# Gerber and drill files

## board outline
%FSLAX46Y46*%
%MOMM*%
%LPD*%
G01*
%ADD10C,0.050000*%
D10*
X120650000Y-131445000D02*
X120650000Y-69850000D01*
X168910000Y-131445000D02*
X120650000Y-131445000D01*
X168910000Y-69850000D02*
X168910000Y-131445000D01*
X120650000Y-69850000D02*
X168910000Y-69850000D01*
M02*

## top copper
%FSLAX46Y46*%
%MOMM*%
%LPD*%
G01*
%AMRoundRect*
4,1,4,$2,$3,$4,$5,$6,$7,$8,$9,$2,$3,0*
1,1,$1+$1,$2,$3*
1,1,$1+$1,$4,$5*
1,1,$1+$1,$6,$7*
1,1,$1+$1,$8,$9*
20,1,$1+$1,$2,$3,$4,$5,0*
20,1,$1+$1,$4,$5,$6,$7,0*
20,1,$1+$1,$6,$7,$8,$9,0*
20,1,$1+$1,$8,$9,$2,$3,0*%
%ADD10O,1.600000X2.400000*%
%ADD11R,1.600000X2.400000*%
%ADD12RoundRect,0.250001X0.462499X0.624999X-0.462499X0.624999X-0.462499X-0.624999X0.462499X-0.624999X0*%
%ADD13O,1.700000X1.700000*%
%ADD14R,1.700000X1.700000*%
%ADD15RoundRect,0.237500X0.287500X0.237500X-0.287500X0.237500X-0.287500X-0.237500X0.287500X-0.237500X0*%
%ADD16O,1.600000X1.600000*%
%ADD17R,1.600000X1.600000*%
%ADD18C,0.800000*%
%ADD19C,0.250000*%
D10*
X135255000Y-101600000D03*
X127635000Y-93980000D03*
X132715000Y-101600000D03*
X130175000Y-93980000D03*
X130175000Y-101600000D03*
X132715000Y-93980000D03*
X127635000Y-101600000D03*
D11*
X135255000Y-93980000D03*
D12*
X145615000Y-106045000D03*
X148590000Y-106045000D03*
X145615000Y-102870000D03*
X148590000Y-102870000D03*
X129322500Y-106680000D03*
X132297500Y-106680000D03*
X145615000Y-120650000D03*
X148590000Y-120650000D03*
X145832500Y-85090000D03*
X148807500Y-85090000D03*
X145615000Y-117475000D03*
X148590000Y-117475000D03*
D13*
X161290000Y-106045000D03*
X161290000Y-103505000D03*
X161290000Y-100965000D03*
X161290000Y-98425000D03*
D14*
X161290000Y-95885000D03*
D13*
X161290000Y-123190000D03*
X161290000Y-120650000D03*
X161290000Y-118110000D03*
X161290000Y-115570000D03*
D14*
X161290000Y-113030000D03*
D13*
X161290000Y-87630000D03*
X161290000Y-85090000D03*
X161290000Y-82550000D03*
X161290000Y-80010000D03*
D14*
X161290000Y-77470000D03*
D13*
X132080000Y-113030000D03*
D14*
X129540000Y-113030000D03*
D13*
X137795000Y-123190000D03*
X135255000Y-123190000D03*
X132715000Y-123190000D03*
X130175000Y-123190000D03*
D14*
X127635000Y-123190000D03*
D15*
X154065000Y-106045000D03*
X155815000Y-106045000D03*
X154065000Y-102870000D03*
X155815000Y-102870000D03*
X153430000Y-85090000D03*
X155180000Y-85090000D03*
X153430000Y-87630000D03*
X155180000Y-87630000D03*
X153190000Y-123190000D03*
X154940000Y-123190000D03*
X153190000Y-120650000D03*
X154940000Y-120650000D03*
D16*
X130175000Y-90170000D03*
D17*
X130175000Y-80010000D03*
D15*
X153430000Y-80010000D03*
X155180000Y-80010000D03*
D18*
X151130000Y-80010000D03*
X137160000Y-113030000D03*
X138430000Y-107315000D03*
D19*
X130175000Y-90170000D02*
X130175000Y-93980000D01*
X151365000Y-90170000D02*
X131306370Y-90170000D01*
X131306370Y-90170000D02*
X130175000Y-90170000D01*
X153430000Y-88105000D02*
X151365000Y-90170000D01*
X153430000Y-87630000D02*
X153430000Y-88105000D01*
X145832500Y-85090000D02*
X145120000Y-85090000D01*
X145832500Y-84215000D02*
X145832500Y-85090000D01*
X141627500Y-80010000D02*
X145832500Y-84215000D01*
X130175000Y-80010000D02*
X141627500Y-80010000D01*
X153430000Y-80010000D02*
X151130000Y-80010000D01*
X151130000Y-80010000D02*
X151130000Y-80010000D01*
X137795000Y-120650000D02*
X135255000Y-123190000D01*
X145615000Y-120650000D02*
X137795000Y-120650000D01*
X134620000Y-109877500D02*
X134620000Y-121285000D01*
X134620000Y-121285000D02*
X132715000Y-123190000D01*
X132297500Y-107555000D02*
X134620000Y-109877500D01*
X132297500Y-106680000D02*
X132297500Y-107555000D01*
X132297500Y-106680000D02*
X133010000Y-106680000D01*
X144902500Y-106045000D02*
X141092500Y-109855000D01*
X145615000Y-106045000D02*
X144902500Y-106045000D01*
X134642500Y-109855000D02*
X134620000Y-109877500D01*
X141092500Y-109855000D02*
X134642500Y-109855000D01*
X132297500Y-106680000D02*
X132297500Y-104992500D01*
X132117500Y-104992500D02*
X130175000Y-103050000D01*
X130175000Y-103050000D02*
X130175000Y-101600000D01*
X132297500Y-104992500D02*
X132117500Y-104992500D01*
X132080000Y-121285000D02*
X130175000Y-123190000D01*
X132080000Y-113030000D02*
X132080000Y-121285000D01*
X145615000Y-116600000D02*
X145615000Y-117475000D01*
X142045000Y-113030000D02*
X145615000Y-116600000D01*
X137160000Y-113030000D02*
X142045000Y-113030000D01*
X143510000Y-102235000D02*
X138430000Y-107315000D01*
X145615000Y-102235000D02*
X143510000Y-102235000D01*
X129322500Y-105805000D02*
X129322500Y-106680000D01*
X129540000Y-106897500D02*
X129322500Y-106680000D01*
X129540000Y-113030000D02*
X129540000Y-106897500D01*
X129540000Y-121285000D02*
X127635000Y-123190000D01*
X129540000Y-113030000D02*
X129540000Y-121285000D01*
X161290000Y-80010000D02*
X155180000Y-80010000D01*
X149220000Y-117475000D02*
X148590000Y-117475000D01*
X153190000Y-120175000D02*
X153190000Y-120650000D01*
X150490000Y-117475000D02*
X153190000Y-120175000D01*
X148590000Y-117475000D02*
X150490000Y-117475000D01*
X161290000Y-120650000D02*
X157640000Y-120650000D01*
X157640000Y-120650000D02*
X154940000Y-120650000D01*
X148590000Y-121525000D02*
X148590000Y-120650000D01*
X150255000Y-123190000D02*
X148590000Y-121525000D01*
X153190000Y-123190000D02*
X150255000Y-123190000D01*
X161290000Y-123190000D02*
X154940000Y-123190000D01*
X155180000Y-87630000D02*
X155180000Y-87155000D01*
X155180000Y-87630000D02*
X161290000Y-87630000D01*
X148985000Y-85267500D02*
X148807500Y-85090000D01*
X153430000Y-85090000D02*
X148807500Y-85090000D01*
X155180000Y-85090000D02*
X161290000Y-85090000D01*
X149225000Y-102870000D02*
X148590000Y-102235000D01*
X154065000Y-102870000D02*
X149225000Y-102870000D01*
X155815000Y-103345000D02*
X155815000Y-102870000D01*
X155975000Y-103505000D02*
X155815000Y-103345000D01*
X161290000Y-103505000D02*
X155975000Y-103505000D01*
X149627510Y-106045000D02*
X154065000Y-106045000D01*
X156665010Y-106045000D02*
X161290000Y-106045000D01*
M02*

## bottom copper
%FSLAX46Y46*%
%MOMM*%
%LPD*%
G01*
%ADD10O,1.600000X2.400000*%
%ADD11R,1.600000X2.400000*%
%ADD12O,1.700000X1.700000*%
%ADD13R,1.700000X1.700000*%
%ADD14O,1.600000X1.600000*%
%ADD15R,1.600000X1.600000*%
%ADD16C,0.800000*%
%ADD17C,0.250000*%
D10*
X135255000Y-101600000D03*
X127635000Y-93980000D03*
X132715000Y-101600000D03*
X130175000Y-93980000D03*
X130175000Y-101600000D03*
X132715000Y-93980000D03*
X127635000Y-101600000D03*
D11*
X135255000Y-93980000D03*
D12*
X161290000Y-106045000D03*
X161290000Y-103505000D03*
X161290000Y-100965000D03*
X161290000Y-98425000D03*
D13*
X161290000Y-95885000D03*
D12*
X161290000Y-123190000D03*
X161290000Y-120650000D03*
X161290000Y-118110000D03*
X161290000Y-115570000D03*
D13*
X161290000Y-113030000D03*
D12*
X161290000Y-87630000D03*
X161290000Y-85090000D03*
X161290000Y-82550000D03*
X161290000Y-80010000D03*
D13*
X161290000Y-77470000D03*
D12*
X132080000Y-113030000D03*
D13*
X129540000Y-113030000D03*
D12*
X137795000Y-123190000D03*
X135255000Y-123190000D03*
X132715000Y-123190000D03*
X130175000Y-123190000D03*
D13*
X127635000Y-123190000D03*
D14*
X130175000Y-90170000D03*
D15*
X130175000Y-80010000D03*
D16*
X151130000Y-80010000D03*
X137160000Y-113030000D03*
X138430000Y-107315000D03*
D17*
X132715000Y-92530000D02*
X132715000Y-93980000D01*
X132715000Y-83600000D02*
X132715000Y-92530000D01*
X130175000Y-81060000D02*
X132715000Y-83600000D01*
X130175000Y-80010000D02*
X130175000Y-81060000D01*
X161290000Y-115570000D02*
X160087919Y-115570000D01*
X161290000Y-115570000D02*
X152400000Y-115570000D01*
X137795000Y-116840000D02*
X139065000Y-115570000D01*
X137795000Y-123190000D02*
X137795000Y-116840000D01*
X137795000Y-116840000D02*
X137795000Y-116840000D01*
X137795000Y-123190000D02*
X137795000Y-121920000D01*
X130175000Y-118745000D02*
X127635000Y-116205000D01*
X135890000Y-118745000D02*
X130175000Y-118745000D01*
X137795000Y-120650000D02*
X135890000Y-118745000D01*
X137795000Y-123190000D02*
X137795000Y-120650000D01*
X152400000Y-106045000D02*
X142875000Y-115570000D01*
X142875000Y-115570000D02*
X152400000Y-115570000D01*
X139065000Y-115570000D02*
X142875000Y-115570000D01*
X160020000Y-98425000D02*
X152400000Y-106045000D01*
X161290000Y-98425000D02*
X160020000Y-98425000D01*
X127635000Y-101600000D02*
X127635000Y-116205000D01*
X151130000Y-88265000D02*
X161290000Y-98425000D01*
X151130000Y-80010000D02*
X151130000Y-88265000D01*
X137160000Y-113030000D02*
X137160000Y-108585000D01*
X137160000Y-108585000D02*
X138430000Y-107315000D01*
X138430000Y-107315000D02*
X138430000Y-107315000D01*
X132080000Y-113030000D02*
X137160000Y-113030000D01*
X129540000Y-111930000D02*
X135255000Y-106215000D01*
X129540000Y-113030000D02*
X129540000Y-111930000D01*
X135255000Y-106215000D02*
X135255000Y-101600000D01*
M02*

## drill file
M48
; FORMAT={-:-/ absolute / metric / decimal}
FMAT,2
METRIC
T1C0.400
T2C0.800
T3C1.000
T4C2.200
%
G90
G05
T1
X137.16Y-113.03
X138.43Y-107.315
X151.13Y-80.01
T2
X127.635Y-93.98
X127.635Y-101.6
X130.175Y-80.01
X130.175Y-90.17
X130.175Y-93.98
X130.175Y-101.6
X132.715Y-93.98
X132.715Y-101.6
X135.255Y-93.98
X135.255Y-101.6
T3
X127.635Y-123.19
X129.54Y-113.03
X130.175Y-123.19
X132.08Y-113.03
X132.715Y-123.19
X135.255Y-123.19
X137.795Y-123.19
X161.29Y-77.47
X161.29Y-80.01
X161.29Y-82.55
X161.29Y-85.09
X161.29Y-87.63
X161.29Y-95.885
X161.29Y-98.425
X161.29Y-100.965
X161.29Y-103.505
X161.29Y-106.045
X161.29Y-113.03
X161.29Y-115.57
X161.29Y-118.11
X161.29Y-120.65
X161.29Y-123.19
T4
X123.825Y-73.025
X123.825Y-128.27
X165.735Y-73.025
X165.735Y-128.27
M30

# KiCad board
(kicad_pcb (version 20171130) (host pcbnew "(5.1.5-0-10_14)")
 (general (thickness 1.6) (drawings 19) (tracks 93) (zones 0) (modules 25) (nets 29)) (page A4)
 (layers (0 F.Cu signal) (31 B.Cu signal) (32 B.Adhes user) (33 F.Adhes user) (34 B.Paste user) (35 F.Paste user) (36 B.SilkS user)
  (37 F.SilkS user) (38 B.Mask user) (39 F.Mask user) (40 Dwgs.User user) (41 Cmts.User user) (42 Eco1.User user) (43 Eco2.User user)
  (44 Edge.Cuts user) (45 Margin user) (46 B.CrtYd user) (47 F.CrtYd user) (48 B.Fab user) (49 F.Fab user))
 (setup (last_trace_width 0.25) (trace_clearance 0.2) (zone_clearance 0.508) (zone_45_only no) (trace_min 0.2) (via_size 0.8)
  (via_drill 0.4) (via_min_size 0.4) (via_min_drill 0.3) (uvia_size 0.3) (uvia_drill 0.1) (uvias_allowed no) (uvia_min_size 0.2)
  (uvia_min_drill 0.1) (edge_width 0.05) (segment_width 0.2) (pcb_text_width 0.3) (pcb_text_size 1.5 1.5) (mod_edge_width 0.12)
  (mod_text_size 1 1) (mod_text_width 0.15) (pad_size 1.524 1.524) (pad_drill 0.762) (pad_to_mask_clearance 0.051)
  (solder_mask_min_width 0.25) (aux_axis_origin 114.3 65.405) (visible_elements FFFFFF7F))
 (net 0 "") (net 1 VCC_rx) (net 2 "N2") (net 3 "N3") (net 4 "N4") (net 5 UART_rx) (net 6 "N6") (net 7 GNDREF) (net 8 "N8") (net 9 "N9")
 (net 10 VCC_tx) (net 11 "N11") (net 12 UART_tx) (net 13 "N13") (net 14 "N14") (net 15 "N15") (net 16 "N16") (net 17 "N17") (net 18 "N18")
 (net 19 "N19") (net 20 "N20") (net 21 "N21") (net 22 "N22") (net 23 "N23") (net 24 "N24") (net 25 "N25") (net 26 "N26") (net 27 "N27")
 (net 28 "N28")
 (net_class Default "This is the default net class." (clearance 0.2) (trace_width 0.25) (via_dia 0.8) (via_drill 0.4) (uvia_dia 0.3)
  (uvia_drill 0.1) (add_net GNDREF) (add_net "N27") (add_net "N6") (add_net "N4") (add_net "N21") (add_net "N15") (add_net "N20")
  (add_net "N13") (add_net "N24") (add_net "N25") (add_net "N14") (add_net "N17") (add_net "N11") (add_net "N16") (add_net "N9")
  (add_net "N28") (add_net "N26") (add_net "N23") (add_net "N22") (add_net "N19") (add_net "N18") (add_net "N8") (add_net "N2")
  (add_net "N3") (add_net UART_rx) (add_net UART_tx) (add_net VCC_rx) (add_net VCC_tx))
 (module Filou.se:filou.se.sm (layer F.Cu) (at 123.825 79.375 90)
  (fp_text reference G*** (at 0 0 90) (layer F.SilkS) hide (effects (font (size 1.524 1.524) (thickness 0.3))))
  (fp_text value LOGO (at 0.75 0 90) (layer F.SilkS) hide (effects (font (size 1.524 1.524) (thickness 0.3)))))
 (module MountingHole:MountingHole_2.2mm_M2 (layer F.Cu) (at 123.825 73.025)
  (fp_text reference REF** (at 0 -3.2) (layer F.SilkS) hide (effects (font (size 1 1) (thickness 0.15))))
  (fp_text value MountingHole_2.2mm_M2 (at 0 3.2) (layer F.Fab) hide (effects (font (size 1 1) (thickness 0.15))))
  (pad 1 np_thru_hole circle (at 0 0) (size 2.2 2.2) (drill 2.2) (layers *.Cu *.Mask)))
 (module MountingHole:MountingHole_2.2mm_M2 (layer F.Cu) (at 165.735 73.025)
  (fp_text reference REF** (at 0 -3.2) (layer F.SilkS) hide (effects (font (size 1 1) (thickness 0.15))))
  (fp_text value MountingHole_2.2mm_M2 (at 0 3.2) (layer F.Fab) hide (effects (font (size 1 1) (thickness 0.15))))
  (pad 1 np_thru_hole circle (at 0 0) (size 2.2 2.2) (drill 2.2) (layers *.Cu *.Mask)))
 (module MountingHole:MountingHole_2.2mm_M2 (layer F.Cu) (at 165.735 128.27)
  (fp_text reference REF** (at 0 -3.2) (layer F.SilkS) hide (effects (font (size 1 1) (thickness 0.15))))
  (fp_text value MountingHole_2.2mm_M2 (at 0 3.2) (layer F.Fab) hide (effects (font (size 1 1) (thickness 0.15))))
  (pad 1 np_thru_hole circle (at 0 0) (size 2.2 2.2) (drill 2.2) (layers *.Cu *.Mask)))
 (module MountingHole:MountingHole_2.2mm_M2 (layer F.Cu) (at 123.825 128.27)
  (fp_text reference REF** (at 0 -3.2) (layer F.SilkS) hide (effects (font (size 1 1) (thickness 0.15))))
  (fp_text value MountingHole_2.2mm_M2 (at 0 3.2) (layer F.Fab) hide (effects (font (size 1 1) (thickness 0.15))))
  (pad 1 np_thru_hole circle (at 0 0) (size 2.2 2.2) (drill 2.2) (layers *.Cu *.Mask)))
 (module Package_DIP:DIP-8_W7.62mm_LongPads (layer F.Cu) (at 135.255 93.98 270)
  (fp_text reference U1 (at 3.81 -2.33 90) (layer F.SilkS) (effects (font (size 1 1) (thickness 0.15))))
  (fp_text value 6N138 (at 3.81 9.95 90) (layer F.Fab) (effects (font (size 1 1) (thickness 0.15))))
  (pad 8 thru_hole oval (at 7.62 0 270) (size 2.4 1.6) (drill 0.8) (layers *.Cu *.Mask) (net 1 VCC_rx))
  (pad 4 thru_hole oval (at 0 7.62 270) (size 2.4 1.6) (drill 0.8) (layers *.Cu *.Mask) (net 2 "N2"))
  (pad 7 thru_hole oval (at 7.62 2.54 270) (size 2.4 1.6) (drill 0.8) (layers *.Cu *.Mask) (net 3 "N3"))
  (pad 3 thru_hole oval (at 0 5.08 270) (size 2.4 1.6) (drill 0.8) (layers *.Cu *.Mask) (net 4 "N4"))
  (pad 6 thru_hole oval (at 7.62 5.08 270) (size 2.4 1.6) (drill 0.8) (layers *.Cu *.Mask) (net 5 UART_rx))
  (pad 2 thru_hole oval (at 0 2.54 270) (size 2.4 1.6) (drill 0.8) (layers *.Cu *.Mask) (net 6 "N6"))
  (pad 5 thru_hole oval (at 7.62 7.62 270) (size 2.4 1.6) (drill 0.8) (layers *.Cu *.Mask) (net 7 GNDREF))
  (pad 1 thru_hole rect (at 0 0 270) (size 2.4 1.6) (drill 0.8) (layers *.Cu *.Mask) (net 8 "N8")))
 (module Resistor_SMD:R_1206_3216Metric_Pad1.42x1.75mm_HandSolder (layer F.Cu) (at 147.1025 106.045 180)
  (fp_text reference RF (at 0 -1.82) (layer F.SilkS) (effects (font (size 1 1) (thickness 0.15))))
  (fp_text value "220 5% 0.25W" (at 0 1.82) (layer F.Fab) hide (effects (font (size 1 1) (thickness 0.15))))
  (pad 2 smd roundrect (at 1.4875 0 180) (size 1.425 1.75) (layers F.Cu F.Paste F.Mask) (roundrect_rratio 0.175439) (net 5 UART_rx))
  (pad 1 smd roundrect (at -1.4875 0 180) (size 1.425 1.75) (layers F.Cu F.Paste F.Mask) (roundrect_rratio 0.175439) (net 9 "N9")))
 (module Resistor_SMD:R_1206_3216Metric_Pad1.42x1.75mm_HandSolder (layer F.Cu) (at 147.1025 102.87 180)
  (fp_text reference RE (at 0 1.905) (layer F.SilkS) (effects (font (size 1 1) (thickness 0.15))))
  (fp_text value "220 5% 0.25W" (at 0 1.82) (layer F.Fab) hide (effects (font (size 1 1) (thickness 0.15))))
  (pad 2 smd roundrect (at 1.4875 0 180) (size 1.425 1.75) (layers F.Cu F.Paste F.Mask) (roundrect_rratio 0.175439) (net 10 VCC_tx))
  (pad 1 smd roundrect (at -1.4875 0 180) (size 1.425 1.75) (layers F.Cu F.Paste F.Mask) (roundrect_rratio 0.175439) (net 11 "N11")))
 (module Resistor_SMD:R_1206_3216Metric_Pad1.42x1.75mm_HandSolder (layer F.Cu) (at 130.81 106.68 180)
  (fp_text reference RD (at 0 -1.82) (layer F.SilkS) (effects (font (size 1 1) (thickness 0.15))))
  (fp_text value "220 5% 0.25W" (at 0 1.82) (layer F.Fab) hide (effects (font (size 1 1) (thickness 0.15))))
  (pad 2 smd roundrect (at 1.4875 0 180) (size 1.425 1.75) (layers F.Cu F.Paste F.Mask) (roundrect_rratio 0.175439) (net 1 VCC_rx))
  (pad 1 smd roundrect (at -1.4875 0 180) (size 1.425 1.75) (layers F.Cu F.Paste F.Mask) (roundrect_rratio 0.175439) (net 5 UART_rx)))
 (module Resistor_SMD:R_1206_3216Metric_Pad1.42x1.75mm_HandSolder (layer F.Cu) (at 147.1025 120.65 180)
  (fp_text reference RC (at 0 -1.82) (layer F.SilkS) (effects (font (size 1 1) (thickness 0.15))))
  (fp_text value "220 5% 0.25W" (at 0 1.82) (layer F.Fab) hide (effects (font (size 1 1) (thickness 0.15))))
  (pad 2 smd roundrect (at 1.4875 0 180) (size 1.425 1.75) (layers F.Cu F.Paste F.Mask) (roundrect_rratio 0.175439) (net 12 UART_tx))
  (pad 1 smd roundrect (at -1.4875 0 180) (size 1.425 1.75) (layers F.Cu F.Paste F.Mask) (roundrect_rratio 0.175439) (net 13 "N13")))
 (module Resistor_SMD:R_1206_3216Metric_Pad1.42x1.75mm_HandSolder (layer F.Cu) (at 147.32 85.09 180)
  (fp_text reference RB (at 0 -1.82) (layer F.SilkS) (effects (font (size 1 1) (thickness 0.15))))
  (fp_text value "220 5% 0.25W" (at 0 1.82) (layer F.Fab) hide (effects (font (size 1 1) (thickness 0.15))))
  (pad 2 smd roundrect (at 1.4875 0 180) (size 1.425 1.75) (layers F.Cu F.Paste F.Mask) (roundrect_rratio 0.175439) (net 6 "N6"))
  (pad 1 smd roundrect (at -1.4875 0 180) (size 1.425 1.75) (layers F.Cu F.Paste F.Mask) (roundrect_rratio 0.175439) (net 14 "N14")))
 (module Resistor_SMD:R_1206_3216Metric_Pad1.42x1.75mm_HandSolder (layer F.Cu) (at 147.1025 117.475 180)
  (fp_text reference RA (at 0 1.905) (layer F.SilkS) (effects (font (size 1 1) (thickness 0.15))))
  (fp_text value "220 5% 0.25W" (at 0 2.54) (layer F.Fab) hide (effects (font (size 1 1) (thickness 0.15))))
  (pad 2 smd roundrect (at 1.4875 0 180) (size 1.425 1.75) (layers F.Cu F.Paste F.Mask) (roundrect_rratio 0.175439) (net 10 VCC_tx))
  (pad 1 smd roundrect (at -1.4875 0 180) (size 1.425 1.75) (layers F.Cu F.Paste F.Mask) (roundrect_rratio 0.175439) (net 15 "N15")))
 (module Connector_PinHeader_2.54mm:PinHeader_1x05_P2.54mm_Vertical (layer F.Cu) (at 161.29 95.885)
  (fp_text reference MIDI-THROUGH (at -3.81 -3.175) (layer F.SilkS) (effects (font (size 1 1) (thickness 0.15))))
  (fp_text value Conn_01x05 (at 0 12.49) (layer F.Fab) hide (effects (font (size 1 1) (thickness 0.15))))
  (pad 5 thru_hole oval (at 0 10.16) (size 1.7 1.7) (drill 1) (layers *.Cu *.Mask) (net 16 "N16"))
  (pad 4 thru_hole oval (at 0 7.62) (size 1.7 1.7) (drill 1) (layers *.Cu *.Mask) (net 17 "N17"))
  (pad 3 thru_hole oval (at 0 5.08) (size 1.7 1.7) (drill 1) (layers *.Cu *.Mask) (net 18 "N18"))
  (pad 2 thru_hole oval (at 0 2.54) (size 1.7 1.7) (drill 1) (layers *.Cu *.Mask) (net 7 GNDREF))
  (pad 1 thru_hole rect (at 0 0) (size 1.7 1.7) (drill 1) (layers *.Cu *.Mask) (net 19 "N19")))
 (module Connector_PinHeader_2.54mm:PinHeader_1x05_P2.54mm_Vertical (layer F.Cu) (at 161.29 113.03)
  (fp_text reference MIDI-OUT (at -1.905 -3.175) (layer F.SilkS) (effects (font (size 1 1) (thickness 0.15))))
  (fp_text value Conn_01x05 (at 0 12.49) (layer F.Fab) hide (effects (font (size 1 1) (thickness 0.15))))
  (pad 5 thru_hole oval (at 0 10.16) (size 1.7 1.7) (drill 1) (layers *.Cu *.Mask) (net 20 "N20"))
  (pad 4 thru_hole oval (at 0 7.62) (size 1.7 1.7) (drill 1) (layers *.Cu *.Mask) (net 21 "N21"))
  (pad 3 thru_hole oval (at 0 5.08) (size 1.7 1.7) (drill 1) (layers *.Cu *.Mask) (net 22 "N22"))
  (pad 2 thru_hole oval (at 0 2.54) (size 1.7 1.7) (drill 1) (layers *.Cu *.Mask) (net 7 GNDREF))
  (pad 1 thru_hole rect (at 0 0) (size 1.7 1.7) (drill 1) (layers *.Cu *.Mask) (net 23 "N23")))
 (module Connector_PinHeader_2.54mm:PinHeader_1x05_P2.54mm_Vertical (layer F.Cu) (at 161.29 77.47)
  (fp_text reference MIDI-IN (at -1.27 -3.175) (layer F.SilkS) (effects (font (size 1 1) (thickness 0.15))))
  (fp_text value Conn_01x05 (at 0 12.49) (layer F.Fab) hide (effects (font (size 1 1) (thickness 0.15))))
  (pad 5 thru_hole oval (at 0 10.16) (size 1.7 1.7) (drill 1) (layers *.Cu *.Mask) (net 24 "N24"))
  (pad 4 thru_hole oval (at 0 7.62) (size 1.7 1.7) (drill 1) (layers *.Cu *.Mask) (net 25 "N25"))
  (pad 3 thru_hole oval (at 0 5.08) (size 1.7 1.7) (drill 1) (layers *.Cu *.Mask) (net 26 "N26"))
  (pad 2 thru_hole oval (at 0 2.54) (size 1.7 1.7) (drill 1) (layers *.Cu *.Mask) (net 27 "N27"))
  (pad 1 thru_hole rect (at 0 0) (size 1.7 1.7) (drill 1) (layers *.Cu *.Mask) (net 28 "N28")))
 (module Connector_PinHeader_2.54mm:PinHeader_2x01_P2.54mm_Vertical (layer F.Cu) (at 129.54 113.03)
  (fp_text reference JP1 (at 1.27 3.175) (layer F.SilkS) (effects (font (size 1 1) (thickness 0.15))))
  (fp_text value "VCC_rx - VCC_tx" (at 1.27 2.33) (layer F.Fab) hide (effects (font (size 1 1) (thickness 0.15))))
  (pad 2 thru_hole oval (at 2.54 0) (size 1.7 1.7) (drill 1) (layers *.Cu *.Mask) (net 10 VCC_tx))
  (pad 1 thru_hole rect (at 0 0) (size 1.7 1.7) (drill 1) (layers *.Cu *.Mask) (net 1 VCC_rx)))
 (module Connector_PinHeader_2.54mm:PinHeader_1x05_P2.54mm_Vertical (layer F.Cu) (at 127.635 123.19 90)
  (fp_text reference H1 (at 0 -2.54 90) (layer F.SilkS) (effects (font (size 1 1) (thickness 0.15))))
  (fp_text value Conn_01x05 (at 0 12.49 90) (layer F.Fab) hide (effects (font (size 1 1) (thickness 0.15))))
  (pad 5 thru_hole oval (at 0 10.16 90) (size 1.7 1.7) (drill 1) (layers *.Cu *.Mask) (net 7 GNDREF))
  (pad 4 thru_hole oval (at 0 7.62 90) (size 1.7 1.7) (drill 1) (layers *.Cu *.Mask) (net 12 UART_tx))
  (pad 3 thru_hole oval (at 0 5.08 90) (size 1.7 1.7) (drill 1) (layers *.Cu *.Mask) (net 5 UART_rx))
  (pad 2 thru_hole oval (at 0 2.54 90) (size 1.7 1.7) (drill 1) (layers *.Cu *.Mask) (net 10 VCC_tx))
  (pad 1 thru_hole rect (at 0 0 90) (size 1.7 1.7) (drill 1) (layers *.Cu *.Mask) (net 1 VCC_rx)))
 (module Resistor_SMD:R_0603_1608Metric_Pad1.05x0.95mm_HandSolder (layer F.Cu) (at 154.94 106.045 180)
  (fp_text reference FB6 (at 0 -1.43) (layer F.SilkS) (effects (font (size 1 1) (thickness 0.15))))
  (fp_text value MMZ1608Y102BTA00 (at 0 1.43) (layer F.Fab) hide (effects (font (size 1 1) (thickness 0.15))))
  (pad 2 smd roundrect (at 0.875 0 180) (size 1.05 0.95) (layers F.Cu F.Paste F.Mask) (roundrect_rratio 0.25) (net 9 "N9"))
  (pad 1 smd roundrect (at -0.875 0 180) (size 1.05 0.95) (layers F.Cu F.Paste F.Mask) (roundrect_rratio 0.25) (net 16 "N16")))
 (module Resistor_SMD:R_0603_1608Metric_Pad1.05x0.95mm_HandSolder (layer F.Cu) (at 154.94 102.87 180)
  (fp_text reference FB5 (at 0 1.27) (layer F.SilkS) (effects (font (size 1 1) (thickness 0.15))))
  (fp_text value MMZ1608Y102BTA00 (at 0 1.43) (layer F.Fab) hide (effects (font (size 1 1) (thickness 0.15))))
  (pad 2 smd roundrect (at 0.875 0 180) (size 1.05 0.95) (layers F.Cu F.Paste F.Mask) (roundrect_rratio 0.25) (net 11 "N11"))
  (pad 1 smd roundrect (at -0.875 0 180) (size 1.05 0.95) (layers F.Cu F.Paste F.Mask) (roundrect_rratio 0.25) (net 17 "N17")))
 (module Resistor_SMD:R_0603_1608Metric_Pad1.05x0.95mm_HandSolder (layer F.Cu) (at 154.305 85.09 180)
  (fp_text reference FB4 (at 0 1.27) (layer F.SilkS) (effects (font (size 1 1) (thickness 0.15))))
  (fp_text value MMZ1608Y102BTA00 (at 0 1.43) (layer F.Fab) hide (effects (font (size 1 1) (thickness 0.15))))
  (pad 2 smd roundrect (at 0.875 0 180) (size 1.05 0.95) (layers F.Cu F.Paste F.Mask) (roundrect_rratio 0.25) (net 14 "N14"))
  (pad 1 smd roundrect (at -0.875 0 180) (size 1.05 0.95) (layers F.Cu F.Paste F.Mask) (roundrect_rratio 0.25) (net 25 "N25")))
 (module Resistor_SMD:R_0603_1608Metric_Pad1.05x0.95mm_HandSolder (layer F.Cu) (at 154.305 87.63 180)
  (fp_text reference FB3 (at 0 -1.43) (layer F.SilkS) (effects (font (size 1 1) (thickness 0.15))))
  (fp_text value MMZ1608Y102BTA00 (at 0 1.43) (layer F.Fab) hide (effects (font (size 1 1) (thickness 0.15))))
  (pad 2 smd roundrect (at 0.875 0 180) (size 1.05 0.95) (layers F.Cu F.Paste F.Mask) (roundrect_rratio 0.25) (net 4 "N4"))
  (pad 1 smd roundrect (at -0.875 0 180) (size 1.05 0.95) (layers F.Cu F.Paste F.Mask) (roundrect_rratio 0.25) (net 24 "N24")))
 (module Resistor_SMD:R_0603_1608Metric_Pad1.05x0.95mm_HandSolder (layer F.Cu) (at 154.065 123.19 180)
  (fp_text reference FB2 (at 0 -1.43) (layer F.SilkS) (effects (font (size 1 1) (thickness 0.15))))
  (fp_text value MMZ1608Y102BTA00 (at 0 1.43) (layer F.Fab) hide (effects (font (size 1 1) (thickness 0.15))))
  (pad 2 smd roundrect (at 0.875 0 180) (size 1.05 0.95) (layers F.Cu F.Paste F.Mask) (roundrect_rratio 0.25) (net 13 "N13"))
  (pad 1 smd roundrect (at -0.875 0 180) (size 1.05 0.95) (layers F.Cu F.Paste F.Mask) (roundrect_rratio 0.25) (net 20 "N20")))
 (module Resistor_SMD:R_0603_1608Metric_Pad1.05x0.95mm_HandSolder (layer F.Cu) (at 154.065 120.65 180)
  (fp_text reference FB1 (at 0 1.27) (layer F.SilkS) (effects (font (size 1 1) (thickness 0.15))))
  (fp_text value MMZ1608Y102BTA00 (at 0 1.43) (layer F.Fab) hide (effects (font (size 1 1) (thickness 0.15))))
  (pad 2 smd roundrect (at 0.875 0 180) (size 1.05 0.95) (layers F.Cu F.Paste F.Mask) (roundrect_rratio 0.25) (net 15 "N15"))
  (pad 1 smd roundrect (at -0.875 0 180) (size 1.05 0.95) (layers F.Cu F.Paste F.Mask) (roundrect_rratio 0.25) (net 21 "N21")))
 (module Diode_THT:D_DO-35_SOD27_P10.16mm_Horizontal (layer F.Cu) (at 130.175 80.01 270)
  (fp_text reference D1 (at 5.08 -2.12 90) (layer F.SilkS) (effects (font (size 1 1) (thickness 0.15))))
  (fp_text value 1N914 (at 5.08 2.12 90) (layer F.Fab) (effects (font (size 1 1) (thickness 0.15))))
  (pad 2 thru_hole oval (at 10.16 0 270) (size 1.6 1.6) (drill 0.8) (layers *.Cu *.Mask) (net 4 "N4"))
  (pad 1 thru_hole rect (at 0 0 270) (size 1.6 1.6) (drill 0.8) (layers *.Cu *.Mask) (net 6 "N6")))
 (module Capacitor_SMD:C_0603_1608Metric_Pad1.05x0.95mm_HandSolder (layer F.Cu) (at 154.305 80.01 180)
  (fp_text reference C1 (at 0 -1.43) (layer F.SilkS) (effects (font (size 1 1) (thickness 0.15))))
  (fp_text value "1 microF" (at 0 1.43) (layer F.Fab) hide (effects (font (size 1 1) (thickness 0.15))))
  (pad 2 smd roundrect (at 0.875 0 180) (size 1.05 0.95) (layers F.Cu F.Paste F.Mask) (roundrect_rratio 0.25) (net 7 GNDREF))
  (pad 1 smd roundrect (at -0.875 0 180) (size 1.05 0.95) (layers F.Cu F.Paste F.Mask) (roundrect_rratio 0.25) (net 27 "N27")))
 (gr_line (start 120.65 131.445) (end 120.65 69.85) (layer Edge.Cuts) (width 0.05))
 (gr_line (start 168.91 131.445) (end 120.65 131.445) (layer Edge.Cuts) (width 0.05))
 (gr_line (start 168.91 69.85) (end 168.91 131.445) (layer Edge.Cuts) (width 0.05))
 (gr_line (start 120.65 69.85) (end 168.91 69.85) (layer Edge.Cuts) (width 0.05))
 (segment (start 130.175 90.17) (end 130.175 93.98) (width 0.25) (layer F.Cu) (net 4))
 (segment (start 151.365 90.17) (end 131.30637 90.17) (width 0.25) (layer F.Cu) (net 4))
 (segment (start 131.30637 90.17) (end 130.175 90.17) (width 0.25) (layer F.Cu) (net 4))
 (segment (start 153.43 88.105) (end 151.365 90.17) (width 0.25) (layer F.Cu) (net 4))
 (segment (start 153.43 87.63) (end 153.43 88.105) (width 0.25) (layer F.Cu) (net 4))
 (segment (start 145.8325 85.09) (end 145.12 85.09) (width 0.25) (layer F.Cu) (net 6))
 (segment (start 145.8325 84.215) (end 145.8325 85.09) (width 0.25) (layer F.Cu) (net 6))
 (segment (start 141.6275 80.01) (end 145.8325 84.215) (width 0.25) (layer F.Cu) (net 6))
 (segment (start 130.175 80.01) (end 141.6275 80.01) (width 0.25) (layer F.Cu) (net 6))
 (segment (start 132.715 92.53) (end 132.715 93.98) (width 0.25) (layer B.Cu) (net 6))
 (segment (start 132.715 83.6) (end 132.715 92.53) (width 0.25) (layer B.Cu) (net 6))
 (segment (start 130.175 81.06) (end 132.715 83.6) (width 0.25) (layer B.Cu) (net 6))
 (segment (start 130.175 80.01) (end 130.175 81.06) (width 0.25) (layer B.Cu) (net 6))
 (segment (start 161.29 115.57) (end 160.087919 115.57) (width 0.25) (layer B.Cu) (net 7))
 (segment (start 161.29 115.57) (end 152.4 115.57) (width 0.25) (layer B.Cu) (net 7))
 (segment (start 137.795 116.84) (end 139.065 115.57) (width 0.25) (layer B.Cu) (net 7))
 (segment (start 137.795 123.19) (end 137.795 116.84) (width 0.25) (layer B.Cu) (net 7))
 (segment (start 137.795 116.84) (end 137.795 116.84) (width 0.25) (layer B.Cu) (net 7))
 (segment (start 137.795 123.19) (end 137.795 121.92) (width 0.25) (layer B.Cu) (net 7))
 (segment (start 130.175 118.745) (end 127.635 116.205) (width 0.25) (layer B.Cu) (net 7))
 (segment (start 135.89 118.745) (end 130.175 118.745) (width 0.25) (layer B.Cu) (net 7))
 (segment (start 137.795 120.65) (end 135.89 118.745) (width 0.25) (layer B.Cu) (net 7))
 (segment (start 137.795 123.19) (end 137.795 120.65) (width 0.25) (layer B.Cu) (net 7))
 (segment (start 152.4 106.045) (end 142.875 115.57) (width 0.25) (layer B.Cu) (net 7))
 (segment (start 142.875 115.57) (end 152.4 115.57) (width 0.25) (layer B.Cu) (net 7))
 (segment (start 139.065 115.57) (end 142.875 115.57) (width 0.25) (layer B.Cu) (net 7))
 (segment (start 160.02 98.425) (end 152.4 106.045) (width 0.25) (layer B.Cu) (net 7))
 (segment (start 161.29 98.425) (end 160.02 98.425) (width 0.25) (layer B.Cu) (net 7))
 (segment (start 127.635 101.6) (end 127.635 116.205) (width 0.25) (layer B.Cu) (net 7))
 (segment (start 153.43 80.01) (end 151.13 80.01) (width 0.25) (layer F.Cu) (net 7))
 (segment (start 151.13 80.01) (end 151.13 80.01) (width 0.25) (layer F.Cu) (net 7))
 (via (at 151.13 80.01) (size 0.8) (drill 0.4) (layers F.Cu B.Cu) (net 7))
 (segment (start 151.13 88.265) (end 161.29 98.425) (width 0.25) (layer B.Cu) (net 7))
 (segment (start 151.13 80.01) (end 151.13 88.265) (width 0.25) (layer B.Cu) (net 7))
 (segment (start 137.795 120.65) (end 135.255 123.19) (width 0.25) (layer F.Cu) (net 12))
 (segment (start 145.615 120.65) (end 137.795 120.65) (width 0.25) (layer F.Cu) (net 12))
 (segment (start 134.62 109.8775) (end 134.62 121.285) (width 0.25) (layer F.Cu) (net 5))
 (segment (start 134.62 121.285) (end 132.715 123.19) (width 0.25) (layer F.Cu) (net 5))
 (segment (start 132.2975 107.555) (end 134.62 109.8775) (width 0.25) (layer F.Cu) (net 5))
 (segment (start 132.2975 106.68) (end 132.2975 107.555) (width 0.25) (layer F.Cu) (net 5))
 (segment (start 132.2975 106.68) (end 133.01 106.68) (width 0.25) (layer F.Cu) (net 5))
 (segment (start 144.9025 106.045) (end 141.0925 109.855) (width 0.25) (layer F.Cu) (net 5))
 (segment (start 145.615 106.045) (end 144.9025 106.045) (width 0.25) (layer F.Cu) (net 5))
 (segment (start 134.6425 109.855) (end 134.62 109.8775) (width 0.25) (layer F.Cu) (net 5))
 (segment (start 141.0925 109.855) (end 134.6425 109.855) (width 0.25) (layer F.Cu) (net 5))
 (segment (start 132.2975 106.68) (end 132.2975 104.9925) (width 0.25) (layer F.Cu) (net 5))
 (segment (start 132.1175 104.9925) (end 130.175 103.05) (width 0.25) (layer F.Cu) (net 5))
 (segment (start 130.175 103.05) (end 130.175 101.6) (width 0.25) (layer F.Cu) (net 5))
 (segment (start 132.2975 104.9925) (end 132.1175 104.9925) (width 0.25) (layer F.Cu) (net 5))
 (segment (start 132.08 121.285) (end 130.175 123.19) (width 0.25) (layer F.Cu) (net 10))
 (segment (start 132.08 113.03) (end 132.08 121.285) (width 0.25) (layer F.Cu) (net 10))
 (via (at 137.16 113.03) (size 0.8) (drill 0.4) (layers F.Cu B.Cu) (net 10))
 (segment (start 145.615 116.6) (end 145.615 117.475) (width 0.25) (layer F.Cu) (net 10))
 (segment (start 142.045 113.03) (end 145.615 116.6) (width 0.25) (layer F.Cu) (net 10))
 (segment (start 137.16 113.03) (end 142.045 113.03) (width 0.25) (layer F.Cu) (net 10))
 (segment (start 137.16 113.03) (end 137.16 108.585) (width 0.25) (layer B.Cu) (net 10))
 (segment (start 137.16 108.585) (end 138.43 107.315) (width 0.25) (layer B.Cu) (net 10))
 (segment (start 138.43 107.315) (end 138.43 107.315) (width 0.25) (layer B.Cu) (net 10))
 (via (at 138.43 107.315) (size 0.8) (drill 0.4) (layers F.Cu B.Cu) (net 10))
 (segment (start 143.51 102.235) (end 138.43 107.315) (width 0.25) (layer F.Cu) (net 10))
 (segment (start 145.615 102.235) (end 143.51 102.235) (width 0.25) (layer F.Cu) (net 10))
 (segment (start 132.08 113.03) (end 137.16 113.03) (width 0.25) (layer B.Cu) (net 10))
 (segment (start 129.3225 105.805) (end 129.3225 106.68) (width 0.25) (layer F.Cu) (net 1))
 (segment (start 129.54 106.8975) (end 129.3225 106.68) (width 0.25) (layer F.Cu) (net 1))
 (segment (start 129.54 113.03) (end 129.54 106.8975) (width 0.25) (layer F.Cu) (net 1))
 (segment (start 129.54 121.285) (end 127.635 123.19) (width 0.25) (layer F.Cu) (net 1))
 (segment (start 129.54 113.03) (end 129.54 121.285) (width 0.25) (layer F.Cu) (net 1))
 (segment (start 129.54 111.93) (end 135.255 106.215) (width 0.25) (layer B.Cu) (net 1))
 (segment (start 129.54 113.03) (end 129.54 111.93) (width 0.25) (layer B.Cu) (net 1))
 (segment (start 135.255 106.215) (end 135.255 101.6) (width 0.25) (layer B.Cu) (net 1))
 (segment (start 161.29 80.01) (end 155.18 80.01) (width 0.25) (layer F.Cu) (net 27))
 (segment (start 149.22 117.475) (end 148.59 117.475) (width 0.25) (layer F.Cu) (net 15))
 (segment (start 153.19 120.175) (end 153.19 120.65) (width 0.25) (layer F.Cu) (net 15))
 (segment (start 150.49 117.475) (end 153.19 120.175) (width 0.25) (layer F.Cu) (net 15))
 (segment (start 148.59 117.475) (end 150.49 117.475) (width 0.25) (layer F.Cu) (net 15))
 (segment (start 161.29 120.65) (end 157.64 120.65) (width 0.25) (layer F.Cu) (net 21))
 (segment (start 157.64 120.65) (end 154.94 120.65) (width 0.25) (layer F.Cu) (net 21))
 (segment (start 148.59 121.525) (end 148.59 120.65) (width 0.25) (layer F.Cu) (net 13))
 (segment (start 150.255 123.19) (end 148.59 121.525) (width 0.25) (layer F.Cu) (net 13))
 (segment (start 153.19 123.19) (end 150.255 123.19) (width 0.25) (layer F.Cu) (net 13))
 (segment (start 161.29 123.19) (end 154.94 123.19) (width 0.25) (layer F.Cu) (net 20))
 (segment (start 155.18 87.63) (end 155.18 87.155) (width 0.25) (layer F.Cu) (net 24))
 (segment (start 155.18 87.63) (end 161.29 87.63) (width 0.25) (layer F.Cu) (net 24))
 (segment (start 148.985 85.2675) (end 148.8075 85.09) (width 0.25) (layer F.Cu) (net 14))
 (segment (start 153.43 85.09) (end 148.8075 85.09) (width 0.25) (layer F.Cu) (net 14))
 (segment (start 155.18 85.09) (end 161.29 85.09) (width 0.25) (layer F.Cu) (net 25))
 (segment (start 149.225 102.87) (end 148.59 102.235) (width 0.25) (layer F.Cu) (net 11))
 (segment (start 154.065 102.87) (end 149.225 102.87) (width 0.25) (layer F.Cu) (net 11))
 (segment (start 155.815 103.345) (end 155.815 102.87) (width 0.25) (layer F.Cu) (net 17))
 (segment (start 155.975 103.505) (end 155.815 103.345) (width 0.25) (layer F.Cu) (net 17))
 (segment (start 161.29 103.505) (end 155.975 103.505) (width 0.25) (layer F.Cu) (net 17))
 (segment (start 149.62751 106.045) (end 154.065 106.045) (width 0.25) (layer F.Cu) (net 9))
 (segment (start 156.66501 106.045) (end 161.29 106.045) (width 0.25) (layer F.Cu) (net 16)))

